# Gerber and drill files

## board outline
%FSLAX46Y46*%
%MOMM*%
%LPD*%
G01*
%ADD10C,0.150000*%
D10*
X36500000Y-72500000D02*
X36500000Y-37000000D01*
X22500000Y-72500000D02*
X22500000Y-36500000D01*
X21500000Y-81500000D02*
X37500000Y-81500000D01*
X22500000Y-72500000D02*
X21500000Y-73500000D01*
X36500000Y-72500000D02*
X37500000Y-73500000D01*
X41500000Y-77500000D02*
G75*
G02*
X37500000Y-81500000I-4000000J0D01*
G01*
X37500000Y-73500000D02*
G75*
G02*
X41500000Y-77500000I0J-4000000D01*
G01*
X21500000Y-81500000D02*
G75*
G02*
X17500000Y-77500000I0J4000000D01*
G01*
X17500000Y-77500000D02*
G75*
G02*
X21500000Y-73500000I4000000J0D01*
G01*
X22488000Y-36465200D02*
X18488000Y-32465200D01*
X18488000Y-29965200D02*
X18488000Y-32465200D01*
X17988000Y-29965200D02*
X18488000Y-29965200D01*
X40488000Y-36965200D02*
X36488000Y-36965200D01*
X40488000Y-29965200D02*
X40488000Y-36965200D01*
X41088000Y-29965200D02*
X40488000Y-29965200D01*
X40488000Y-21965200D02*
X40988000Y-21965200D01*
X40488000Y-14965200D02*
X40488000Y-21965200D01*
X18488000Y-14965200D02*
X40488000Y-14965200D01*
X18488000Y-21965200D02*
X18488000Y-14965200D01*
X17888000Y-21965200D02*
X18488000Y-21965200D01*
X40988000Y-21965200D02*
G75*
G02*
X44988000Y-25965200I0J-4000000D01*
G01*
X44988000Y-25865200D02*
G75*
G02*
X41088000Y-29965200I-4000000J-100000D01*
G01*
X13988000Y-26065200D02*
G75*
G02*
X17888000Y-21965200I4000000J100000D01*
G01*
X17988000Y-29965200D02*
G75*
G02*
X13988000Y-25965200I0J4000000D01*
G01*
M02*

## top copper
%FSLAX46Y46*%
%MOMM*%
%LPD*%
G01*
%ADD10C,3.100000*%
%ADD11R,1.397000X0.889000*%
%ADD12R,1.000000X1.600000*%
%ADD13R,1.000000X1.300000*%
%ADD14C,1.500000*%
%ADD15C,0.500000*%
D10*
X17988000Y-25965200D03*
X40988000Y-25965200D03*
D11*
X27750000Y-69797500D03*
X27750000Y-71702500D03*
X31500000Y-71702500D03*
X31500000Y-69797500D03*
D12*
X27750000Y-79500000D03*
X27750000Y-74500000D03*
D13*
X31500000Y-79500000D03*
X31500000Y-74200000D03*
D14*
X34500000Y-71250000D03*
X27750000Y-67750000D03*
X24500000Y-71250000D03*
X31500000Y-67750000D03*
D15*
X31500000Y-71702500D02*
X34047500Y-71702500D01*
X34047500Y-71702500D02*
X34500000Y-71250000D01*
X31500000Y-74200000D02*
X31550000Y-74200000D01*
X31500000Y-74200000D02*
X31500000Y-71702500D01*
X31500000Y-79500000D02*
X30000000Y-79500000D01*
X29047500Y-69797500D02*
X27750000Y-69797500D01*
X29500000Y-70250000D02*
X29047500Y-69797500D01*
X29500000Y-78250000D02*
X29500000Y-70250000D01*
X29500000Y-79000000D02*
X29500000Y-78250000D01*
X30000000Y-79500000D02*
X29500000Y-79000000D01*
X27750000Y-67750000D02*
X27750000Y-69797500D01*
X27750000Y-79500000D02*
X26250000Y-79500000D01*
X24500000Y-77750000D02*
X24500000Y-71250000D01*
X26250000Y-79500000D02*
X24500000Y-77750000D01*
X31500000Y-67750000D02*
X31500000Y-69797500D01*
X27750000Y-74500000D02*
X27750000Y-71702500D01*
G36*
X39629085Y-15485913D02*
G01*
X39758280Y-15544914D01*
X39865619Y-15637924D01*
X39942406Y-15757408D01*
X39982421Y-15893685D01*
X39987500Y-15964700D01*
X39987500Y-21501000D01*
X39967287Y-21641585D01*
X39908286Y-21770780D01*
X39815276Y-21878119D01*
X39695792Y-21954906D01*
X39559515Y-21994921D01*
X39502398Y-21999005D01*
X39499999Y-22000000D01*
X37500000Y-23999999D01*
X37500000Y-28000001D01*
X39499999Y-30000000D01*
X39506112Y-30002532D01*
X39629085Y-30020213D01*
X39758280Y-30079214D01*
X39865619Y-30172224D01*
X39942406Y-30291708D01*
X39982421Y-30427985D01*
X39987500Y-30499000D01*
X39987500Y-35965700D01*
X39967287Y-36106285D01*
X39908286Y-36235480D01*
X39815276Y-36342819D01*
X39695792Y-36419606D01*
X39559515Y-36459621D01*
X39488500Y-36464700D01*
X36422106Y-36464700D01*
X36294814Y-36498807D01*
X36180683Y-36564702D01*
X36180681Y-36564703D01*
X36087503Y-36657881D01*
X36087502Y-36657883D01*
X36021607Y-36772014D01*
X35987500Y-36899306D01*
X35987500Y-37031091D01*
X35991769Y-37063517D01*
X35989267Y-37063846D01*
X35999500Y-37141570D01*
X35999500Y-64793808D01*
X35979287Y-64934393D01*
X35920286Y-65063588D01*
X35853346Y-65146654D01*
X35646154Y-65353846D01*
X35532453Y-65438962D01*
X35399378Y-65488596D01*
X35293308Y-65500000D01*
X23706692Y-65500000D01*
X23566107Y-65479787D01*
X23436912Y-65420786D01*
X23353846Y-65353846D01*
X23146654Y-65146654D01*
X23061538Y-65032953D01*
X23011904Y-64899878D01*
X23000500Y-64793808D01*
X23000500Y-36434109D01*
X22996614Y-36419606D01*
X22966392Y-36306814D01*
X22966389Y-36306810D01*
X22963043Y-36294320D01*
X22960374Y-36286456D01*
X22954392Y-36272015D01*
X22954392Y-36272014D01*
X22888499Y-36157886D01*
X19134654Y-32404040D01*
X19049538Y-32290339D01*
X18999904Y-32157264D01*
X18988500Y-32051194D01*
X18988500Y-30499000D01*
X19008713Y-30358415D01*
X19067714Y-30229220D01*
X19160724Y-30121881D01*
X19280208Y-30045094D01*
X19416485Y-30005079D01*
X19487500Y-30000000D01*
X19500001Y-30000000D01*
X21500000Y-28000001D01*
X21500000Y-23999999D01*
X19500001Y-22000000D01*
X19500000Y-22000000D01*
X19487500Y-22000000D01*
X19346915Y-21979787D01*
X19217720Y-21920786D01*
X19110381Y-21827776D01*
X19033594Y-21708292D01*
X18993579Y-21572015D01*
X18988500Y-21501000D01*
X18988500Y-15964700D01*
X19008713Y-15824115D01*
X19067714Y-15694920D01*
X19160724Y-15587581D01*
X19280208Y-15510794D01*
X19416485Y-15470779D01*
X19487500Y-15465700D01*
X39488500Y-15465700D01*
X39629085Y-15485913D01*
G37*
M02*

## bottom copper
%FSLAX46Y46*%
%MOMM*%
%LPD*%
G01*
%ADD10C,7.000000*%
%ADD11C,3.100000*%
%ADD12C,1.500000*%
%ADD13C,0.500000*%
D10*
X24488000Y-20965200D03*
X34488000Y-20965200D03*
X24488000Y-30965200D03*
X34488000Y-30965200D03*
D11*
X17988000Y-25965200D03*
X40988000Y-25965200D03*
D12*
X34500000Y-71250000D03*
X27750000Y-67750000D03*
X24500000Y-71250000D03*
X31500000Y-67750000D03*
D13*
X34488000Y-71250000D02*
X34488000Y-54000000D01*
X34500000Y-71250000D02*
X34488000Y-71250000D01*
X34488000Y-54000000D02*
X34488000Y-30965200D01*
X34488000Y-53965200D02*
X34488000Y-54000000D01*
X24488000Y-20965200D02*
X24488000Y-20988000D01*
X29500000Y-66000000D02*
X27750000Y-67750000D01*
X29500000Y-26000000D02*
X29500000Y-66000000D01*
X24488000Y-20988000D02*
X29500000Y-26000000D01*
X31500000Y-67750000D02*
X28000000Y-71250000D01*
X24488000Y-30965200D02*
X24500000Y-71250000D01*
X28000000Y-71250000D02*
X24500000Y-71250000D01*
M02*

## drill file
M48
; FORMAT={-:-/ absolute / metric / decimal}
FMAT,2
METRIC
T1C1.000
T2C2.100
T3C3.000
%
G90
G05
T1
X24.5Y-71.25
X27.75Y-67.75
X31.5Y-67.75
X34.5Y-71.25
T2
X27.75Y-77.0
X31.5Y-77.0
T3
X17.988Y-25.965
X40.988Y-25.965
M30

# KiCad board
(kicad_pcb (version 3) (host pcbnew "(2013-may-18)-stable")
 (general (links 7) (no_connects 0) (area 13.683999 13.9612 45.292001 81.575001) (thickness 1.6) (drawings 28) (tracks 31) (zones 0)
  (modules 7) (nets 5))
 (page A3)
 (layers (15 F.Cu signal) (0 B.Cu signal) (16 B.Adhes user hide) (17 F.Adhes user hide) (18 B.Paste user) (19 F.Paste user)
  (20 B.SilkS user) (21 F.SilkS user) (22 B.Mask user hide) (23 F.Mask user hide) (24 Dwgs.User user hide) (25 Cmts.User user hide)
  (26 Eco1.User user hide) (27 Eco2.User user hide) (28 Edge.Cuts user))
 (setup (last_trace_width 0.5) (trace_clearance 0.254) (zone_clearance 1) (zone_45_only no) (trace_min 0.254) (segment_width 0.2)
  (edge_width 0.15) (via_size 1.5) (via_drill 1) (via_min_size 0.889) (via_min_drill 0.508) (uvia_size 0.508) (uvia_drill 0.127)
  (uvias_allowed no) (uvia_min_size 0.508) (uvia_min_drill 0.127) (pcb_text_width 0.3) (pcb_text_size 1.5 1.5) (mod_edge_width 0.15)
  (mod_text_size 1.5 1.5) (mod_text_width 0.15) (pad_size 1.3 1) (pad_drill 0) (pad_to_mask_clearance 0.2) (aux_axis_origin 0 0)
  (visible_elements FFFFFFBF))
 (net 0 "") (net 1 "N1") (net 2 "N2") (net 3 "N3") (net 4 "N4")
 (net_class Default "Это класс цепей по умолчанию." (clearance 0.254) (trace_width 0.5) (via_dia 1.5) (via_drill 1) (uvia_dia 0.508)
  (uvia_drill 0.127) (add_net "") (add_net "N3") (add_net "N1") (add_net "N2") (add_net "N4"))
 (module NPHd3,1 (layer F.Cu) (at 21.5 76.5)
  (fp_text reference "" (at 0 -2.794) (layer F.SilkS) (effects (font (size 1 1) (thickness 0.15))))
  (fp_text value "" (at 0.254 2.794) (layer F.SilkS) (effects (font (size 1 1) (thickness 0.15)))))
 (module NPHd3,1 (layer F.Cu) (at 37.5 76.5)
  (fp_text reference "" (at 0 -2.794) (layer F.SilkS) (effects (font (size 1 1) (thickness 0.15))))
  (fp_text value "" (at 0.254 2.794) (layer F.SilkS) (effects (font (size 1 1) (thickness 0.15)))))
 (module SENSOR (layer B.Cu) (at 17.988 14.4652)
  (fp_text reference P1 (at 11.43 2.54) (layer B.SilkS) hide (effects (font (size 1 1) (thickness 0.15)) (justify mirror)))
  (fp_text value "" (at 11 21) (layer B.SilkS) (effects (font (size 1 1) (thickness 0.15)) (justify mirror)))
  (pad 2 smd circle (at 6.5 6.5) (size 7 7) (layers B.Cu B.Mask) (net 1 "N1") (solder_mask_margin 0.1))
  (pad 3 smd circle (at 16.5 6.5) (size 7 7) (layers B.Cu B.Mask))
  (pad 1 smd circle (at 6.5 16.5) (size 7 7) (layers B.Cu B.Mask) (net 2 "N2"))
  (pad 4 smd circle (at 16.5 16.5) (size 7 7) (layers B.Cu B.Mask) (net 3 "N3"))
  (pad "" np_thru_hole circle (at 0 11.5) (size 3.1 3.1) (drill 3) (layers *.Cu *.Mask B.SilkS))
  (pad "" np_thru_hole circle (at 23 11.5) (size 3.1 3.1) (drill 3) (layers *.Cu *.Mask B.SilkS)))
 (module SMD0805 (layer F.Cu) (at 27.75 70.75 270)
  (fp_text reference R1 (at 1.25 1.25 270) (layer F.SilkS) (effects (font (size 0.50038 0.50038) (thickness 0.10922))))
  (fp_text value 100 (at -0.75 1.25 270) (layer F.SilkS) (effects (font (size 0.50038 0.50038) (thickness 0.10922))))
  (pad 1 smd rect (at -0.9525 0 270) (size 0.889 1.397) (layers F.Cu F.Paste F.Mask) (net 1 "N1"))
  (pad 2 smd rect (at 0.9525 0 270) (size 0.889 1.397) (layers F.Cu F.Paste F.Mask) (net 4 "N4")))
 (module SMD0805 (layer F.Cu) (at 31.5 70.75 90)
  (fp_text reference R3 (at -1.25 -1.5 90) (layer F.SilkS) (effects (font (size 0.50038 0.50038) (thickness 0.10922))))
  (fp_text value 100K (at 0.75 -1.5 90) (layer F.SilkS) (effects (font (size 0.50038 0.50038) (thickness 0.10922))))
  (pad 1 smd rect (at -0.9525 0 90) (size 0.889 1.397) (layers F.Cu F.Paste F.Mask) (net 3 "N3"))
  (pad 2 smd rect (at 0.9525 0 90) (size 0.889 1.397) (layers F.Cu F.Paste F.Mask) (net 2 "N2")))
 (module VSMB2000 (layer F.Cu) (at 27.75 77 90)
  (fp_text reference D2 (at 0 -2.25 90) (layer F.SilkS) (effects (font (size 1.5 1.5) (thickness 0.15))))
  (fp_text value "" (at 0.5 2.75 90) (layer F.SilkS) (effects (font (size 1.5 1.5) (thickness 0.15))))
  (pad 2 smd rect (at -2.5 0 90) (size 1.6 1) (layers F.Cu F.Paste F.Mask) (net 2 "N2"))
  (pad 1 smd rect (at 2.5 0 90) (size 1.6 1) (layers F.Cu F.Paste F.Mask) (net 4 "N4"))
  (pad "" np_thru_hole circle (at 0 0 90) (size 2.1 2.1) (drill 2.1) (layers *.Cu *.Mask F.SilkS)))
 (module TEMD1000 (layer F.Cu) (at 31.5 77 90)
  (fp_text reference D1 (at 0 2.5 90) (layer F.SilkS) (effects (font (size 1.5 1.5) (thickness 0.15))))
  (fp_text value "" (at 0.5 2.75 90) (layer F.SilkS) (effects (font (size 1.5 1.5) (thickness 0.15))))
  (pad 2 smd rect (at -2.5 0 90) (size 1.3 1) (layers F.Cu F.Paste F.Mask) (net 1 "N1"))
  (pad 1 smd rect (at 2.8 0 90) (size 1.3 1) (layers F.Cu F.Paste F.Mask) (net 3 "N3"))
  (pad "" np_thru_hole circle (at 0 0 90) (size 2.1 2.1) (drill 2.1) (layers *.Cu *.Mask F.SilkS)))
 (gr_line (start 36.5 72.5) (end 36.5 37) (angle 90) (layer Edge.Cuts) (width 0.15))
 (gr_line (start 22.5 72.5) (end 22.5 36.5) (angle 90) (layer Edge.Cuts) (width 0.15))
 (gr_line (start 21.5 81.5) (end 37.5 81.5) (angle 90) (layer Edge.Cuts) (width 0.15))
 (gr_line (start 22.5 72.5) (end 21.5 73.5) (angle 90) (layer Edge.Cuts) (width 0.15))
 (gr_line (start 36.5 72.5) (end 37.5 73.5) (angle 90) (layer Edge.Cuts) (width 0.15))
 (gr_arc (start 37.5 77.5) (end 41.5 77.5) (angle 90) (layer Edge.Cuts) (width 0.15))
 (gr_arc (start 37.5 77.5) (end 37.5 73.5) (angle 90) (layer Edge.Cuts) (width 0.15))
 (gr_arc (start 21.5 77.5) (end 21.5 81.5) (angle 90) (layer Edge.Cuts) (width 0.15))
 (gr_arc (start 21.5 77.5) (end 17.5 77.5) (angle 90) (layer Edge.Cuts) (width 0.15))
 (gr_line (start 22.488 36.4652) (end 18.488 32.4652) (angle 90) (layer Edge.Cuts) (width 0.15))
 (gr_line (start 18.488 29.9652) (end 18.488 32.4652) (angle 90) (layer Edge.Cuts) (width 0.15))
 (gr_line (start 17.988 29.9652) (end 18.488 29.9652) (angle 90) (layer Edge.Cuts) (width 0.15))
 (gr_line (start 40.488 36.9652) (end 36.488 36.9652) (angle 90) (layer Edge.Cuts) (width 0.15))
 (gr_line (start 40.488 29.9652) (end 40.488 36.9652) (angle 90) (layer Edge.Cuts) (width 0.15))
 (gr_line (start 41.088 29.9652) (end 40.488 29.9652) (angle 90) (layer Edge.Cuts) (width 0.15))
 (gr_line (start 40.488 21.9652) (end 40.988 21.9652) (angle 90) (layer Edge.Cuts) (width 0.15))
 (gr_line (start 40.488 14.9652) (end 40.488 21.9652) (angle 90) (layer Edge.Cuts) (width 0.15))
 (gr_line (start 18.488 14.9652) (end 40.488 14.9652) (angle 90) (layer Edge.Cuts) (width 0.15))
 (gr_line (start 18.488 21.9652) (end 18.488 14.9652) (angle 90) (layer Edge.Cuts) (width 0.15))
 (gr_line (start 17.888 21.9652) (end 18.488 21.9652) (angle 90) (layer Edge.Cuts) (width 0.15))
 (gr_arc (start 40.988 25.9652) (end 44.988 25.9652) (angle -90) (layer Edge.Cuts) (width 0.15))
 (gr_arc (start 40.988 25.9652) (end 41.088 29.9652) (angle -90) (layer Edge.Cuts) (width 0.15))
 (gr_arc (start 17.988 25.9652) (end 17.888 21.9652) (angle -90) (layer Edge.Cuts) (width 0.15))
 (gr_arc (start 17.988 25.9652) (end 13.988 25.9652) (angle -90) (layer Edge.Cuts) (width 0.15))
 (segment (start 31.5 71.7025) (end 34.0475 71.7025) (width 0.5) (layer F.Cu) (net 3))
 (segment (start 34.488 71.25) (end 34.488 54) (width 0.5) (layer B.Cu) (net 3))
 (segment (start 34.5 71.25) (end 34.488 71.25) (width 0.5) (layer B.Cu) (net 3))
 (via (at 34.5 71.25) (size 1.5) (layers F.Cu B.Cu) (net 3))
 (segment (start 34.0475 71.7025) (end 34.5 71.25) (width 0.5) (layer F.Cu) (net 3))
 (segment (start 31.5 74.2) (end 31.55 74.2) (width 0.5) (layer F.Cu) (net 3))
 (segment (start 31.5 74.2) (end 31.5 71.7025) (width 0.5) (layer F.Cu) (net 3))
 (segment (start 34.488 54) (end 34.488 30.9652) (width 0.5) (layer B.Cu) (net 3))
 (segment (start 34.488 53.9652) (end 34.488 54) (width 0.5) (layer B.Cu) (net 3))
 (segment (start 31.5 79.5) (end 30 79.5) (width 0.5) (layer F.Cu) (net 1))
 (segment (start 29.0475 69.7975) (end 27.75 69.7975) (width 0.5) (layer F.Cu) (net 1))
 (segment (start 29.5 70.25) (end 29.0475 69.7975) (width 0.5) (layer F.Cu) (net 1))
 (segment (start 29.5 78.25) (end 29.5 70.25) (width 0.5) (layer F.Cu) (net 1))
 (segment (start 29.5 79) (end 29.5 78.25) (width 0.5) (layer F.Cu) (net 1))
 (segment (start 30 79.5) (end 29.5 79) (width 0.5) (layer F.Cu) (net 1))
 (segment (start 24.488 20.9652) (end 24.488 20.988) (width 0.5) (layer B.Cu) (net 1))
 (via (at 27.75 67.75) (size 1.5) (layers F.Cu B.Cu) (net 1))
 (segment (start 27.75 67.75) (end 27.75 69.7975) (width 0.5) (layer F.Cu) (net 1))
 (segment (start 29.5 66) (end 27.75 67.75) (width 0.5) (layer B.Cu) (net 1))
 (segment (start 29.5 26) (end 29.5 66) (width 0.5) (layer B.Cu) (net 1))
 (segment (start 24.488 20.988) (end 29.5 26) (width 0.5) (layer B.Cu) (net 1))
 (segment (start 27.75 79.5) (end 26.25 79.5) (width 0.5) (layer F.Cu) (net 2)) (via (at 24.5 71.25) (size 1.5) (layers F.Cu B.Cu) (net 2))
 (segment (start 24.5 77.75) (end 24.5 71.25) (width 0.5) (layer F.Cu) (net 2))
 (segment (start 26.25 79.5) (end 24.5 77.75) (width 0.5) (layer F.Cu) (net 2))
 (segment (start 31.5 67.75) (end 28 71.25) (width 0.5) (layer B.Cu) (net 2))
 (segment (start 24.488 30.9652) (end 24.5 71.25) (width 0.5) (layer B.Cu) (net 2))
 (via (at 31.5 67.75) (size 1.5) (layers F.Cu B.Cu) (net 2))
 (segment (start 31.5 67.75) (end 31.5 69.7975) (width 0.5) (layer F.Cu) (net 2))
 (segment (start 28 71.25) (end 24.5 71.25) (width 0.5) (layer B.Cu) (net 2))
 (segment (start 27.75 74.5) (end 27.75 71.7025) (width 0.5) (layer F.Cu) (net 4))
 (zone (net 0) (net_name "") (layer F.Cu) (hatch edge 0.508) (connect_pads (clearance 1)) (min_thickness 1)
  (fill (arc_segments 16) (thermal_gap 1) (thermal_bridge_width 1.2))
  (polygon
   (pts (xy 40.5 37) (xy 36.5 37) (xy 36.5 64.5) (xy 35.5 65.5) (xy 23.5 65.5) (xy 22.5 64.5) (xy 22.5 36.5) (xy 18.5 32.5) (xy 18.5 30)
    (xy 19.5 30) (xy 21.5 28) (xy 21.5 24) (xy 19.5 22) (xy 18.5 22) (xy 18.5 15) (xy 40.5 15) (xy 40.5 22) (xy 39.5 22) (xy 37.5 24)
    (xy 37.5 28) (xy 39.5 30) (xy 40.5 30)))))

